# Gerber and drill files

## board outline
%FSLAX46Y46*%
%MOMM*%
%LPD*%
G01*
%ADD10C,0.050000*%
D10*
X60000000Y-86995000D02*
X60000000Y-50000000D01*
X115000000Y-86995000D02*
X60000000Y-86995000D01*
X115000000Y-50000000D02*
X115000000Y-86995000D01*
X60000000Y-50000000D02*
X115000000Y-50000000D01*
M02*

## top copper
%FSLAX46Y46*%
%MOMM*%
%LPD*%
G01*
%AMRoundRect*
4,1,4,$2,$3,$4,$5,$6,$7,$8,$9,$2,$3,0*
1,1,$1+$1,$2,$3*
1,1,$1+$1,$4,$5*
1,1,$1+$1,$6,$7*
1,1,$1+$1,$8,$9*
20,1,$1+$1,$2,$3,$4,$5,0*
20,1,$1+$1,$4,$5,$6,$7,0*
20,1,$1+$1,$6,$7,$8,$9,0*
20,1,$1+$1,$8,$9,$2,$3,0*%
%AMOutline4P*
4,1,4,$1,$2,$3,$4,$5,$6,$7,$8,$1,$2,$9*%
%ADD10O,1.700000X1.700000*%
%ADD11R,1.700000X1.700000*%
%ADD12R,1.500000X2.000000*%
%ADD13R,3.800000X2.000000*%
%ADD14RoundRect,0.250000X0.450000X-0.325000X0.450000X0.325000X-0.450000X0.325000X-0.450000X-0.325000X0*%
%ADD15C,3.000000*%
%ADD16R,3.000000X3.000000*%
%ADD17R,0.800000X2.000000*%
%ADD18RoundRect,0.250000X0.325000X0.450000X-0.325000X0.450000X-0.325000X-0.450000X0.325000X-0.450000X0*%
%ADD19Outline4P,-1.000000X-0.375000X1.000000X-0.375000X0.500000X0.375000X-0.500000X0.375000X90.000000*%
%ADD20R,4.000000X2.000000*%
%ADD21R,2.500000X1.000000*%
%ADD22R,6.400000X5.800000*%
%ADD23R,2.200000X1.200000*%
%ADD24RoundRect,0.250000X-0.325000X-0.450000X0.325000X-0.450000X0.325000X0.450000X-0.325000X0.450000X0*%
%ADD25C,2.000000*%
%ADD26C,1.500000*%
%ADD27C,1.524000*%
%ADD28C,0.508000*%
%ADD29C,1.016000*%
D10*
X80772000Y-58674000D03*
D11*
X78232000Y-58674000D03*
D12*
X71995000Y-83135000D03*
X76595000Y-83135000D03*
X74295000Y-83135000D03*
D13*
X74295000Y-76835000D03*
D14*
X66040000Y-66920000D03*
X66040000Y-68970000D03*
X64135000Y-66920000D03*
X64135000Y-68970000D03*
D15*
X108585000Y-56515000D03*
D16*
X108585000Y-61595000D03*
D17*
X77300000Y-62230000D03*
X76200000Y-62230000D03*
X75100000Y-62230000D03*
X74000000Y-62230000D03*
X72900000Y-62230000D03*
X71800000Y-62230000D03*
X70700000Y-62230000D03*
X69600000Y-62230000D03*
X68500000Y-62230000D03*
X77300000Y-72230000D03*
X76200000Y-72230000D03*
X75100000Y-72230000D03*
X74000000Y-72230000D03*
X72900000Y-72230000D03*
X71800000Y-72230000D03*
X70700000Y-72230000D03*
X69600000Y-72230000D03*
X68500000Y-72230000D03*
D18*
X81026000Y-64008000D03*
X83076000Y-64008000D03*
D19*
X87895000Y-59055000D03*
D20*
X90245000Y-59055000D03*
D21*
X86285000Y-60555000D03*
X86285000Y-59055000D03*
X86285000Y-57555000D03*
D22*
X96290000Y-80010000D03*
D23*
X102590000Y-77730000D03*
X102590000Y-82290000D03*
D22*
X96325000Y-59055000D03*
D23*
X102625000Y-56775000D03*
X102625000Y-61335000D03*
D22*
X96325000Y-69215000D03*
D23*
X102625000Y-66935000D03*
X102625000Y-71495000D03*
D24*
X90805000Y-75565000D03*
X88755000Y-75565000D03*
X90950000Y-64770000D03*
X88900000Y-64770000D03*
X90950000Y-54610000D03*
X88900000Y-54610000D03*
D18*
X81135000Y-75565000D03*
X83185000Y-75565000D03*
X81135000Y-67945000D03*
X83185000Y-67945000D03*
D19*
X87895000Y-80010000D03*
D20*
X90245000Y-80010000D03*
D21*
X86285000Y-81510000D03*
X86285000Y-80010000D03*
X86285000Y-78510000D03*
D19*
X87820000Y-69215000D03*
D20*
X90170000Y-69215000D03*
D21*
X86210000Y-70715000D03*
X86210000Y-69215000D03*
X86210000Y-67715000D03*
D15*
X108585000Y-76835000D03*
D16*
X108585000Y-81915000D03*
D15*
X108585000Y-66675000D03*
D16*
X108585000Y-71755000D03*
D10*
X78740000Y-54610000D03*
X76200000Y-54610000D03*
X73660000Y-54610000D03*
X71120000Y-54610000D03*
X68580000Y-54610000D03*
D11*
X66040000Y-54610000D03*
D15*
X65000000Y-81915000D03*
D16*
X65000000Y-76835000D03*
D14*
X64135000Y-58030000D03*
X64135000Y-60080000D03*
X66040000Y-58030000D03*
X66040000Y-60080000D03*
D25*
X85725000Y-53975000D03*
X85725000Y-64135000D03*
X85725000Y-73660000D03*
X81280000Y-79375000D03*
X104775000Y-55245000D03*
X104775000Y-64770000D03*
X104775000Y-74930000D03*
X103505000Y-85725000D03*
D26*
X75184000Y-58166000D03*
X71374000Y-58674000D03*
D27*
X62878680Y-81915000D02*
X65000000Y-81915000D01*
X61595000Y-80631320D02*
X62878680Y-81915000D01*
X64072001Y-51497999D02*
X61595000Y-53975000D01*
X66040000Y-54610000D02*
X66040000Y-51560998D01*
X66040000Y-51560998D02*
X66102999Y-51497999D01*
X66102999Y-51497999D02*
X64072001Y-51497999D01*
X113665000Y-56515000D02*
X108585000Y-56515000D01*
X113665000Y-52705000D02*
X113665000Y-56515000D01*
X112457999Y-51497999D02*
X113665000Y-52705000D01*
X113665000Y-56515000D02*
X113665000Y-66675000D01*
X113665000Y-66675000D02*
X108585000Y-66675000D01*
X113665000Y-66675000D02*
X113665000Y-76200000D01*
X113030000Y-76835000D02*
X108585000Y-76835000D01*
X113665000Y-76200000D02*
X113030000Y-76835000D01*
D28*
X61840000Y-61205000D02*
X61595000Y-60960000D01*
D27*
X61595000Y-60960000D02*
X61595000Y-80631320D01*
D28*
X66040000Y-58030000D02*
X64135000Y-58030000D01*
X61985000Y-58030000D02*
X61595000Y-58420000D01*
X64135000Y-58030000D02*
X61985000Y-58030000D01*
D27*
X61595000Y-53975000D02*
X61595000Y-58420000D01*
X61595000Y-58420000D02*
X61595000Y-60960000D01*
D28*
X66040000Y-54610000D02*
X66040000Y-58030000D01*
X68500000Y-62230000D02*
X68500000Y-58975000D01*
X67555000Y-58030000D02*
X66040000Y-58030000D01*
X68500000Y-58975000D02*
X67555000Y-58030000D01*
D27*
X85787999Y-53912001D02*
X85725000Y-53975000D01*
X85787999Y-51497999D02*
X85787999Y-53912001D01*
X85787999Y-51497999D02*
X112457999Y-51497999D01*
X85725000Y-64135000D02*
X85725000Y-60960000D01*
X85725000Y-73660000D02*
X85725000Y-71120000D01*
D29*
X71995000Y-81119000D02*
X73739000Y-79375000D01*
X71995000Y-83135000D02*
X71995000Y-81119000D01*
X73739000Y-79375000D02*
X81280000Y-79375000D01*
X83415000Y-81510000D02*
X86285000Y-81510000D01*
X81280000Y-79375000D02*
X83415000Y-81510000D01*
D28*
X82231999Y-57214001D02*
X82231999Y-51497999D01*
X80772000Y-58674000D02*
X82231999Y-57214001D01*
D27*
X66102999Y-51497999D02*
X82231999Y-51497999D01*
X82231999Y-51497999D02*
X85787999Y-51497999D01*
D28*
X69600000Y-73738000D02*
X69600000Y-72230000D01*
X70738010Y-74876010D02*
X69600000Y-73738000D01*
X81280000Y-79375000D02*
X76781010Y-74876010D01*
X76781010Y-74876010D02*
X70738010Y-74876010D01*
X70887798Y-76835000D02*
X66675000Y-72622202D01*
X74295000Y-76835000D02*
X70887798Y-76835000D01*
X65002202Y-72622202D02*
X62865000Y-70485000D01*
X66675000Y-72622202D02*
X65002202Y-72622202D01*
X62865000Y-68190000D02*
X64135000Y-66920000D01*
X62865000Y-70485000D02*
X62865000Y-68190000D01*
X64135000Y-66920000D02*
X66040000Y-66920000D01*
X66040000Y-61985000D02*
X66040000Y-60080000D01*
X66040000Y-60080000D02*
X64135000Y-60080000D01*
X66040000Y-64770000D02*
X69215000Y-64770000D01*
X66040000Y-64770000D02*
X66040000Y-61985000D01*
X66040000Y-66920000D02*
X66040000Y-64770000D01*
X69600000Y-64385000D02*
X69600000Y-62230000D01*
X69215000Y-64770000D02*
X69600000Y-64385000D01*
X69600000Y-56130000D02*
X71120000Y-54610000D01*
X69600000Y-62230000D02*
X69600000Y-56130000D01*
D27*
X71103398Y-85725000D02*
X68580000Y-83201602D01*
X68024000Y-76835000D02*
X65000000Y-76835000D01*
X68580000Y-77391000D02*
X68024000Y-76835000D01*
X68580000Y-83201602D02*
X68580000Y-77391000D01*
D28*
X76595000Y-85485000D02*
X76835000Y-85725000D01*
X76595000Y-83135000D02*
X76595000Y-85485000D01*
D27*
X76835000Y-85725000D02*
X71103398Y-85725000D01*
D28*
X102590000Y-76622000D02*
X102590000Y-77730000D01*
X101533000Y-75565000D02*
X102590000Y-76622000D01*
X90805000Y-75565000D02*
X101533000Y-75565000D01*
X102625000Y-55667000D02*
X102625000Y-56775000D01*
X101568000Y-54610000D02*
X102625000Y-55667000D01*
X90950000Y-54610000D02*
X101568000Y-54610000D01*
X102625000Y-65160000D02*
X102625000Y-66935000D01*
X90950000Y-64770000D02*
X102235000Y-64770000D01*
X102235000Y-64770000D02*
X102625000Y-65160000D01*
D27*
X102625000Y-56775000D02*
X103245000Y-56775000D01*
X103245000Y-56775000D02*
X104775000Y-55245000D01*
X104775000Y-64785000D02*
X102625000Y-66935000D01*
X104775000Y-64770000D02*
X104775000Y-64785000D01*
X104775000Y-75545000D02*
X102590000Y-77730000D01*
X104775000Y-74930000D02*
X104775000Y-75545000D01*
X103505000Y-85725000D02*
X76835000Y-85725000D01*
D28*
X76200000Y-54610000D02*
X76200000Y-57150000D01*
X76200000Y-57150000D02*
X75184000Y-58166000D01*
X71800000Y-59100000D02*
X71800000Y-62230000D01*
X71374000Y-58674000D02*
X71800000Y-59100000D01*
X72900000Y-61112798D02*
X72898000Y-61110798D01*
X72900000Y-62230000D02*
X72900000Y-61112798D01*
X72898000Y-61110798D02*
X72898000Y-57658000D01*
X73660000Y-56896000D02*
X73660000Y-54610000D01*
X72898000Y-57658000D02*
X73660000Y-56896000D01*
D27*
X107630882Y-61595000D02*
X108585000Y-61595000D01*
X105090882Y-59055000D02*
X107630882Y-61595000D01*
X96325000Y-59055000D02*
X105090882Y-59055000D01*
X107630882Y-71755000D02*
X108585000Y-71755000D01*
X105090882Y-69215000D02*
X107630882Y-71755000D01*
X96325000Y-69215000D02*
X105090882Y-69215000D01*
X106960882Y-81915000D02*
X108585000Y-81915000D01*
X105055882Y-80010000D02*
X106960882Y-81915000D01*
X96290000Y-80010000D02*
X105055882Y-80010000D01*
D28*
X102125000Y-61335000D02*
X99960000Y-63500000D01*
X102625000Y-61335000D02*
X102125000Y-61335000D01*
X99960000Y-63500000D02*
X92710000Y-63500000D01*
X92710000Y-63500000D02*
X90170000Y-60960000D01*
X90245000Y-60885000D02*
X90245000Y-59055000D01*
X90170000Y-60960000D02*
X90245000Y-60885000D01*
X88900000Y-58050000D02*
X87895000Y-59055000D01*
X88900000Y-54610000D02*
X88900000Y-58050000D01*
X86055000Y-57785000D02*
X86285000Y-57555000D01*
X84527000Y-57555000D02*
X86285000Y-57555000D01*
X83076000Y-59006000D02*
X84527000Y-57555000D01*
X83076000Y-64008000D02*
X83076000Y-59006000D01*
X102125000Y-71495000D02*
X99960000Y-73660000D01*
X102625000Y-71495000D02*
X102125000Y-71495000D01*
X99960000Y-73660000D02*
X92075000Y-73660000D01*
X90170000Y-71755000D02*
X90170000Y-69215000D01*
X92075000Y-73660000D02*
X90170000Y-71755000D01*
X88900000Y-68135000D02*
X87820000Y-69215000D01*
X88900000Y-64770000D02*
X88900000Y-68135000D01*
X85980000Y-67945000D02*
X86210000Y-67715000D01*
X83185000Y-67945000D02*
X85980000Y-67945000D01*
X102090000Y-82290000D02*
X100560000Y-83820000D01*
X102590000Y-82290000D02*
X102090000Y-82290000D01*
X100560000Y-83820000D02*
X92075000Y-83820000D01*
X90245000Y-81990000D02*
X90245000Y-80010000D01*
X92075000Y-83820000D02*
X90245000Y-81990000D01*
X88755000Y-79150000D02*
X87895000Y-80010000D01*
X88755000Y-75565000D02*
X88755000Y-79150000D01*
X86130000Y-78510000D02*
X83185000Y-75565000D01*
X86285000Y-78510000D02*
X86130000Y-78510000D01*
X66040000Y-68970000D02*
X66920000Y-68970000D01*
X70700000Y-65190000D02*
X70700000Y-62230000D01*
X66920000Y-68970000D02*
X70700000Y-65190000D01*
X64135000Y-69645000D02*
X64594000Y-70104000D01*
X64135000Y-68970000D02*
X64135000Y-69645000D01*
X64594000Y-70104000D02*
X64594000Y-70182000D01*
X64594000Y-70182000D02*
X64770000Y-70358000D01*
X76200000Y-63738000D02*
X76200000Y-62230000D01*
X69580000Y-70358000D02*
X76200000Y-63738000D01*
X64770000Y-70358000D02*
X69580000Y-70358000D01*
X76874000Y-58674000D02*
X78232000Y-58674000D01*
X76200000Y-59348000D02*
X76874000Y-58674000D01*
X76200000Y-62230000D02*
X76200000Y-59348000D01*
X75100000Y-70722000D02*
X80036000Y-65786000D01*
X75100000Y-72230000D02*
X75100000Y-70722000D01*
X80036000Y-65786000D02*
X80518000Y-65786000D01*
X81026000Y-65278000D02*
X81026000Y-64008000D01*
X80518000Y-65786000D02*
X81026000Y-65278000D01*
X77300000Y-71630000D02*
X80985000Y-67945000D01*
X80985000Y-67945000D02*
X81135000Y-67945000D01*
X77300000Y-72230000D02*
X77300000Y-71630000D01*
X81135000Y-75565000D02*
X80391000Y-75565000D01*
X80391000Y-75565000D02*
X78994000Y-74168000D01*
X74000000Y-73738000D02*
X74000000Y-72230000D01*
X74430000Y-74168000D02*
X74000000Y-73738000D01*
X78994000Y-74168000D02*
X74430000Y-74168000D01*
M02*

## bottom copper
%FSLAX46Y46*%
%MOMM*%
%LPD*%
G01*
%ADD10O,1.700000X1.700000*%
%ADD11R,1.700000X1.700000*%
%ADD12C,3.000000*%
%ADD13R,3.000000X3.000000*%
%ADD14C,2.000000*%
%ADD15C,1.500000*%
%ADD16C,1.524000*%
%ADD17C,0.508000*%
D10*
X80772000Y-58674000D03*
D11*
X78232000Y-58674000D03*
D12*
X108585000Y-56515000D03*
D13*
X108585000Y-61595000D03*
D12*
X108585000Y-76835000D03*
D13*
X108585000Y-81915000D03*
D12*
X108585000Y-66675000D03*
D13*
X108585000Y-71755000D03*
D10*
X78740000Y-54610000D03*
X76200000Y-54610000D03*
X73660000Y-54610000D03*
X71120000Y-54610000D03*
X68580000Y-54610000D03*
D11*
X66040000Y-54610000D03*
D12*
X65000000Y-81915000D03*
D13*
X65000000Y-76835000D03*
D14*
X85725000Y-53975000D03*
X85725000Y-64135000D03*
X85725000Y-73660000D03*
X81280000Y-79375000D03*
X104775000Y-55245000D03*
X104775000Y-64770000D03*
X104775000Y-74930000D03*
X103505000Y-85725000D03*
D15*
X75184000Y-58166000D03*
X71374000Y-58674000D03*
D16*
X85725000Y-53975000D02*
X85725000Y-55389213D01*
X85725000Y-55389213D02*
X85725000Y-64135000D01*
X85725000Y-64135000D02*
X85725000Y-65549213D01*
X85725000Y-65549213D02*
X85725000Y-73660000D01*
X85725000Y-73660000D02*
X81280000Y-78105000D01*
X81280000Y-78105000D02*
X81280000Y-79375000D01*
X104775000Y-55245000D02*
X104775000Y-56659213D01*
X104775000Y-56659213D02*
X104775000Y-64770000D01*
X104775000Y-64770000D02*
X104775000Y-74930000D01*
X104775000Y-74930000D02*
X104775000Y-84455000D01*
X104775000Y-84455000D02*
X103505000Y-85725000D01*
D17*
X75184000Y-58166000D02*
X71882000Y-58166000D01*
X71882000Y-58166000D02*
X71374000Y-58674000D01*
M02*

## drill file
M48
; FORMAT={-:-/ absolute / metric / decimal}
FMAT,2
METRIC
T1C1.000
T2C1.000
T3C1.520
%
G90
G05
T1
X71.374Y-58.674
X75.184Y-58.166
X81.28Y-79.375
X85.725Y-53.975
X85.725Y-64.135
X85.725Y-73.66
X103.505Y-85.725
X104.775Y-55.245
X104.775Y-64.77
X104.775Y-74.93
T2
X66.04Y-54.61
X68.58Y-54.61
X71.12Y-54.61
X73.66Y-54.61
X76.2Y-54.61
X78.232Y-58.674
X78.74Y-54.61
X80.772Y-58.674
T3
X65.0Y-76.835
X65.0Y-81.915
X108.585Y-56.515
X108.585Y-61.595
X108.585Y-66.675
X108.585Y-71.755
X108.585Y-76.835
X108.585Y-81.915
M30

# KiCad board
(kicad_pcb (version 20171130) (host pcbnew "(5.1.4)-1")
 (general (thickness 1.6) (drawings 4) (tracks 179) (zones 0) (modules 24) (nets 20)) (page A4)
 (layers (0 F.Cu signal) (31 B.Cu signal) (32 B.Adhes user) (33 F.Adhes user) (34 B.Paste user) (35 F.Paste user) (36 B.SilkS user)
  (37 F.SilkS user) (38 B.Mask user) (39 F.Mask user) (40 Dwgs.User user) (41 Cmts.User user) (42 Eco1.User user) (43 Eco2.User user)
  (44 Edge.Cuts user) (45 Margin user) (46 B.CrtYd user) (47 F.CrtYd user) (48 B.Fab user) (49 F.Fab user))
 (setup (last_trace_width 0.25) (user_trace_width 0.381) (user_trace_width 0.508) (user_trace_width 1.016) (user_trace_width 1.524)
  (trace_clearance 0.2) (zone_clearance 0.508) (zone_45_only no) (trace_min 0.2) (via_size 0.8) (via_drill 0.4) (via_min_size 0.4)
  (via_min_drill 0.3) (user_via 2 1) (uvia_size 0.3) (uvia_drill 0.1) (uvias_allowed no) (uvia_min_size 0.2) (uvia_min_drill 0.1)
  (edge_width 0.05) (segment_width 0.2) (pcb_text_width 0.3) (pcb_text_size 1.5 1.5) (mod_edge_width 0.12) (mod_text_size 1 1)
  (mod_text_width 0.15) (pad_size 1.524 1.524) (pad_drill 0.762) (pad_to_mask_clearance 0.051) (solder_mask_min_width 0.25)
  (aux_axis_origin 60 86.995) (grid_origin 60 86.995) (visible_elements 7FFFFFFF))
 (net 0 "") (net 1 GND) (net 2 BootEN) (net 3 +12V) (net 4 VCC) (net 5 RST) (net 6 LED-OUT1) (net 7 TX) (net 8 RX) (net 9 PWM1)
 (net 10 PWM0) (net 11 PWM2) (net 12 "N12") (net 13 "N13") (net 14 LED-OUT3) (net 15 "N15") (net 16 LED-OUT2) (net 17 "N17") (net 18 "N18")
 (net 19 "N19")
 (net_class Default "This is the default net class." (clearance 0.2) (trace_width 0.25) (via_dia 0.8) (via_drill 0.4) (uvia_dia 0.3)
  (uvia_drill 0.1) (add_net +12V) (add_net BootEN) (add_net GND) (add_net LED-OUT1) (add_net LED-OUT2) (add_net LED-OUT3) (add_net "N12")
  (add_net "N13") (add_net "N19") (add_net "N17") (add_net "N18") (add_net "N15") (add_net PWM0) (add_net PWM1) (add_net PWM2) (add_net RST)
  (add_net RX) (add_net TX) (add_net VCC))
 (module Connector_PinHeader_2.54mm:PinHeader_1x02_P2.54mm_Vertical (layer F.Cu) (at 78.232 58.674 90)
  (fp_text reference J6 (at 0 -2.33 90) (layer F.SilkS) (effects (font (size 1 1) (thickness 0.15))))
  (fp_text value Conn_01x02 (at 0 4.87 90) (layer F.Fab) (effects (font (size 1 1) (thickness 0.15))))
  (pad 2 thru_hole oval (at 0 2.54 90) (size 1.7 1.7) (drill 1) (layers *.Cu *.Mask) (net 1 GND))
  (pad 1 thru_hole rect (at 0 0 90) (size 1.7 1.7) (drill 1) (layers *.Cu *.Mask) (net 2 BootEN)))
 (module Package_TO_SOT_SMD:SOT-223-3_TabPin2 (layer F.Cu) (at 74.295 79.985 90)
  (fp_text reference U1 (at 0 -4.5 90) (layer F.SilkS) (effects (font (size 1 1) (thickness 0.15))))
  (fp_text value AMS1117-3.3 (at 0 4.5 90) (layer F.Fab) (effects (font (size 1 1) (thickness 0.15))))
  (pad 1 smd rect (at -3.15 -2.3 90) (size 2 1.5) (layers F.Cu F.Paste F.Mask) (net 1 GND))
  (pad 3 smd rect (at -3.15 2.3 90) (size 2 1.5) (layers F.Cu F.Paste F.Mask) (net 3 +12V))
  (pad 2 smd rect (at -3.15 0 90) (size 2 1.5) (layers F.Cu F.Paste F.Mask) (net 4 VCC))
  (pad 2 smd rect (at 3.15 0 90) (size 2 3.8) (layers F.Cu F.Paste F.Mask) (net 4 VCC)))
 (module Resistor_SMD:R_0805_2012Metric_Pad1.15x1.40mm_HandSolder (layer F.Cu) (at 66.04 67.945 90)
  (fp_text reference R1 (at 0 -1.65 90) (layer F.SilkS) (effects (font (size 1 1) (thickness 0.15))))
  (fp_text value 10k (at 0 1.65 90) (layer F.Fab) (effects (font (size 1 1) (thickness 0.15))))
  (pad 2 smd roundrect (at 1.025 0 90) (size 1.15 1.4) (layers F.Cu F.Paste F.Mask) (roundrect_rratio 0.217391) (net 4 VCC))
  (pad 1 smd roundrect (at -1.025 0 90) (size 1.15 1.4) (layers F.Cu F.Paste F.Mask) (roundrect_rratio 0.217391) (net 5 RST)))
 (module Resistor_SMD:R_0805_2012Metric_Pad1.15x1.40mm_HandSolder (layer F.Cu) (at 64.135 67.945 90)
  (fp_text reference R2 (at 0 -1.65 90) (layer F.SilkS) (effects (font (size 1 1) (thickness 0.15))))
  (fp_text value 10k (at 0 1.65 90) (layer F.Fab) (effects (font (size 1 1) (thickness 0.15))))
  (pad 2 smd roundrect (at 1.025 0 90) (size 1.15 1.4) (layers F.Cu F.Paste F.Mask) (roundrect_rratio 0.217391) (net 4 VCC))
  (pad 1 smd roundrect (at -1.025 0 90) (size 1.15 1.4) (layers F.Cu F.Paste F.Mask) (roundrect_rratio 0.217391) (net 2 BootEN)))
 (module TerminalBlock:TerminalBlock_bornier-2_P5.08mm (layer F.Cu) (at 108.585 61.595 90)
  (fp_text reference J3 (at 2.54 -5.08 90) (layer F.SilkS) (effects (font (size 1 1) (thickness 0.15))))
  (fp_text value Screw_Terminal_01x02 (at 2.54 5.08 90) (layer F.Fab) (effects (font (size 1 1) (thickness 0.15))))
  (pad 2 thru_hole circle (at 5.08 0 90) (size 3 3) (drill 1.52) (layers *.Cu *.Mask) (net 1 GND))
  (pad 1 thru_hole rect (at 0 0 90) (size 3 3) (drill 1.52) (layers *.Cu *.Mask) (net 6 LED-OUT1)))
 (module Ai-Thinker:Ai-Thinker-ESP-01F (layer F.Cu) (at 72.4 67.23 90)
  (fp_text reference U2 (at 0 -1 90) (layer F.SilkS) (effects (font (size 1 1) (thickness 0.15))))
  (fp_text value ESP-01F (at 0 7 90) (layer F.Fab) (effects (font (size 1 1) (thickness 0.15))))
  (pad 18 smd rect (at 5 4.9 90) (size 2 0.8) (layers F.Cu F.Paste F.Mask))
  (pad 17 smd rect (at 5 3.8 90) (size 2 0.8) (layers F.Cu F.Paste F.Mask) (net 2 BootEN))
  (pad 16 smd rect (at 5 2.7 90) (size 2 0.8) (layers F.Cu F.Paste F.Mask))
  (pad 15 smd rect (at 5 1.6 90) (size 2 0.8) (layers F.Cu F.Paste F.Mask))
  (pad 14 smd rect (at 5 0.5 90) (size 2 0.8) (layers F.Cu F.Paste F.Mask) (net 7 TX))
  (pad 13 smd rect (at 5 -0.6 90) (size 2 0.8) (layers F.Cu F.Paste F.Mask) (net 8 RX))
  (pad 12 smd rect (at 5 -1.7 90) (size 2 0.8) (layers F.Cu F.Paste F.Mask) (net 5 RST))
  (pad 11 smd rect (at 5 -2.8 90) (size 2 0.8) (layers F.Cu F.Paste F.Mask) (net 4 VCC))
  (pad 10 smd rect (at 5 -3.9 90) (size 2 0.8) (layers F.Cu F.Paste F.Mask) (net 1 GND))
  (pad 9 smd rect (at -5 4.9 90) (size 2 0.8) (layers F.Cu F.Paste F.Mask) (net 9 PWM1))
  (pad 8 smd rect (at -5 3.8 90) (size 2 0.8) (layers F.Cu F.Paste F.Mask))
  (pad 7 smd rect (at -5 2.7 90) (size 2 0.8) (layers F.Cu F.Paste F.Mask) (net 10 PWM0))
  (pad 6 smd rect (at -5 1.6 90) (size 2 0.8) (layers F.Cu F.Paste F.Mask) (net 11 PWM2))
  (pad 5 smd rect (at -5 0.5 90) (size 2 0.8) (layers F.Cu F.Paste F.Mask))
  (pad 4 smd rect (at -5 -0.6 90) (size 2 0.8) (layers F.Cu F.Paste F.Mask))
  (pad 3 smd rect (at -5 -1.7 90) (size 2 0.8) (layers F.Cu F.Paste F.Mask))
  (pad 2 smd rect (at -5 -2.8 90) (size 2 0.8) (layers F.Cu F.Paste F.Mask) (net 1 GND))
  (pad 1 smd rect (at -5 -3.9 90) (size 2 0.8) (layers F.Cu F.Paste F.Mask)))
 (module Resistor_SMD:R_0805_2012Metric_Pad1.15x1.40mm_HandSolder (layer F.Cu) (at 82.051 64.008 180)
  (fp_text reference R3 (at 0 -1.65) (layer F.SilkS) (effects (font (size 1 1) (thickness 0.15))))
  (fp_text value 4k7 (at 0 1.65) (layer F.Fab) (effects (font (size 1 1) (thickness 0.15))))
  (pad 2 smd roundrect (at 1.025 0 180) (size 1.15 1.4) (layers F.Cu F.Paste F.Mask) (roundrect_rratio 0.217391) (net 10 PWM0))
  (pad 1 smd roundrect (at -1.025 0 180) (size 1.15 1.4) (layers F.Cu F.Paste F.Mask) (roundrect_rratio 0.217391) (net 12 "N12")))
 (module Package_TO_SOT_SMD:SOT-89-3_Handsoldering (layer F.Cu) (at 88.265 59.055)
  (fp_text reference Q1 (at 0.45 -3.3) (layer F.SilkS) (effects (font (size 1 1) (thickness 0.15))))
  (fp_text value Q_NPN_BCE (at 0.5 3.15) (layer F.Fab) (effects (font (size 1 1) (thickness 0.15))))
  (pad 2 smd trapezoid (at -0.37 0 90) (size 1.5 0.75) (rect_delta 0 0.5) (layers F.Cu F.Paste F.Mask) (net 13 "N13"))
  (pad 2 smd rect (at 1.98 0 270) (size 2 4) (layers F.Cu F.Paste F.Mask) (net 13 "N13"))
  (pad 3 smd rect (at -1.98 1.5 270) (size 1 2.5) (layers F.Cu F.Paste F.Mask) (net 1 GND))
  (pad 2 smd rect (at -1.98 0 270) (size 1 2.5) (layers F.Cu F.Paste F.Mask) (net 13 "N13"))
  (pad 1 smd rect (at -1.98 -1.5 270) (size 1 2.5) (layers F.Cu F.Paste F.Mask) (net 12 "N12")))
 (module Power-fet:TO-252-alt (layer F.Cu) (at 98.39 80.01 180)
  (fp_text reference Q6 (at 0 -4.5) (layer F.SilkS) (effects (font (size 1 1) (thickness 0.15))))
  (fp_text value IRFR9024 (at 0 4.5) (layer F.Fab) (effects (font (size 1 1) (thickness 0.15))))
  (pad "" smd rect (at 0.425 1.525 180) (size 3.05 2.75) (layers F.Paste))
  (pad "" smd rect (at 3.775 -1.525 180) (size 3.05 2.75) (layers F.Paste))
  (pad "" smd rect (at 0.425 -1.525 180) (size 3.05 2.75) (layers F.Paste))
  (pad "" smd rect (at 3.775 1.525 180) (size 3.05 2.75) (layers F.Paste))
  (pad 3 smd rect (at 2.1 0 180) (size 6.4 5.8) (layers F.Cu F.Mask) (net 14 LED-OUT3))
  (pad 1 smd rect (at -4.2 2.28 180) (size 2.2 1.2) (layers F.Cu F.Paste F.Mask) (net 3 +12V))
  (pad 2 smd rect (at -4.2 -2.28 180) (size 2.2 1.2) (layers F.Cu F.Paste F.Mask) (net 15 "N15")))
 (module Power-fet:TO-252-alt (layer F.Cu) (at 98.425 59.055 180)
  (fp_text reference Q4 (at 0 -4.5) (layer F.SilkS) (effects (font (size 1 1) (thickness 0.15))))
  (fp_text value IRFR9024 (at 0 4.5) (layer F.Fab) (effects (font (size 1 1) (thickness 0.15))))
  (pad "" smd rect (at 0.425 1.525 180) (size 3.05 2.75) (layers F.Paste))
  (pad "" smd rect (at 3.775 -1.525 180) (size 3.05 2.75) (layers F.Paste))
  (pad "" smd rect (at 0.425 -1.525 180) (size 3.05 2.75) (layers F.Paste))
  (pad "" smd rect (at 3.775 1.525 180) (size 3.05 2.75) (layers F.Paste))
  (pad 3 smd rect (at 2.1 0 180) (size 6.4 5.8) (layers F.Cu F.Mask) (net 6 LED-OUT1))
  (pad 1 smd rect (at -4.2 2.28 180) (size 2.2 1.2) (layers F.Cu F.Paste F.Mask) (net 3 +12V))
  (pad 2 smd rect (at -4.2 -2.28 180) (size 2.2 1.2) (layers F.Cu F.Paste F.Mask) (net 13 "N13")))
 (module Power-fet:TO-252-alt (layer F.Cu) (at 98.425 69.215 180)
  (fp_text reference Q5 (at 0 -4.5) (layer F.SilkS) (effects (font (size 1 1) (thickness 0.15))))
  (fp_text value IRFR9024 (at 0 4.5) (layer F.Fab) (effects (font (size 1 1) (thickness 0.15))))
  (pad "" smd rect (at 0.425 1.525 180) (size 3.05 2.75) (layers F.Paste))
  (pad "" smd rect (at 3.775 -1.525 180) (size 3.05 2.75) (layers F.Paste))
  (pad "" smd rect (at 0.425 -1.525 180) (size 3.05 2.75) (layers F.Paste))
  (pad "" smd rect (at 3.775 1.525 180) (size 3.05 2.75) (layers F.Paste))
  (pad 3 smd rect (at 2.1 0 180) (size 6.4 5.8) (layers F.Cu F.Mask) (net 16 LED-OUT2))
  (pad 1 smd rect (at -4.2 2.28 180) (size 2.2 1.2) (layers F.Cu F.Paste F.Mask) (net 3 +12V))
  (pad 2 smd rect (at -4.2 -2.28 180) (size 2.2 1.2) (layers F.Cu F.Paste F.Mask) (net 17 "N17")))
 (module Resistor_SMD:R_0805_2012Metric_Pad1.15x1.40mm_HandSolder (layer F.Cu) (at 89.78 75.565)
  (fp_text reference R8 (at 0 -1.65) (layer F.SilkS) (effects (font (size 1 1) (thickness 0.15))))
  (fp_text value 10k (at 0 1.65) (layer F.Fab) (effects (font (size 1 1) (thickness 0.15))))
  (pad 2 smd roundrect (at 1.025 0) (size 1.15 1.4) (layers F.Cu F.Paste F.Mask) (roundrect_rratio 0.217391) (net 3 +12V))
  (pad 1 smd roundrect (at -1.025 0) (size 1.15 1.4) (layers F.Cu F.Paste F.Mask) (roundrect_rratio 0.217391) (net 15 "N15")))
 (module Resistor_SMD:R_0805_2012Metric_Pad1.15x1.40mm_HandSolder (layer F.Cu) (at 89.925 64.77)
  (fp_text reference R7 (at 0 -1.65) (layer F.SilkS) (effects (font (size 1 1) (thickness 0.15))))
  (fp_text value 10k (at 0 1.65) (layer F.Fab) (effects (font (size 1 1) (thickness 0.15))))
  (pad 2 smd roundrect (at 1.025 0) (size 1.15 1.4) (layers F.Cu F.Paste F.Mask) (roundrect_rratio 0.217391) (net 3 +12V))
  (pad 1 smd roundrect (at -1.025 0) (size 1.15 1.4) (layers F.Cu F.Paste F.Mask) (roundrect_rratio 0.217391) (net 17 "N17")))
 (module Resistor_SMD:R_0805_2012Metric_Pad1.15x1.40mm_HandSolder (layer F.Cu) (at 89.925 54.61)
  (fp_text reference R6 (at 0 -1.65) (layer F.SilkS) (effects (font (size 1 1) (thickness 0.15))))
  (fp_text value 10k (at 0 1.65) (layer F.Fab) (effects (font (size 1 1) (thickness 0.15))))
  (pad 2 smd roundrect (at 1.025 0) (size 1.15 1.4) (layers F.Cu F.Paste F.Mask) (roundrect_rratio 0.217391) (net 3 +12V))
  (pad 1 smd roundrect (at -1.025 0) (size 1.15 1.4) (layers F.Cu F.Paste F.Mask) (roundrect_rratio 0.217391) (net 13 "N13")))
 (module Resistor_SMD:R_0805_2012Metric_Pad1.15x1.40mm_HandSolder (layer F.Cu) (at 82.16 75.565 180)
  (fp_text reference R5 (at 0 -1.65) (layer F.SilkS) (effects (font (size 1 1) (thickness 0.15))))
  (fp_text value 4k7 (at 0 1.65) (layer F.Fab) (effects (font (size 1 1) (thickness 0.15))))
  (pad 2 smd roundrect (at 1.025 0 180) (size 1.15 1.4) (layers F.Cu F.Paste F.Mask) (roundrect_rratio 0.217391) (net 11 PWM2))
  (pad 1 smd roundrect (at -1.025 0 180) (size 1.15 1.4) (layers F.Cu F.Paste F.Mask) (roundrect_rratio 0.217391) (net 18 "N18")))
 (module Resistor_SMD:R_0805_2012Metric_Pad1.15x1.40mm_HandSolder (layer F.Cu) (at 82.16 67.945 180)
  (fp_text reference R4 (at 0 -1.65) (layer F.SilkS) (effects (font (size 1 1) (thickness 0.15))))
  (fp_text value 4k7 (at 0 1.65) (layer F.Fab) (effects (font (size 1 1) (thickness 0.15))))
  (pad 2 smd roundrect (at 1.025 0 180) (size 1.15 1.4) (layers F.Cu F.Paste F.Mask) (roundrect_rratio 0.217391) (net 9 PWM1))
  (pad 1 smd roundrect (at -1.025 0 180) (size 1.15 1.4) (layers F.Cu F.Paste F.Mask) (roundrect_rratio 0.217391) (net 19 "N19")))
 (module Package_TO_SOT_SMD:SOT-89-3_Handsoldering (layer F.Cu) (at 88.265 80.01)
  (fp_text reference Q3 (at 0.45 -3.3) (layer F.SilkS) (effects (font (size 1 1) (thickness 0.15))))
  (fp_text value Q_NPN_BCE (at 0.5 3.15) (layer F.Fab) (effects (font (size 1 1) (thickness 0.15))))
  (pad 2 smd trapezoid (at -0.37 0 90) (size 1.5 0.75) (rect_delta 0 0.5) (layers F.Cu F.Paste F.Mask) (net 15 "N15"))
  (pad 2 smd rect (at 1.98 0 270) (size 2 4) (layers F.Cu F.Paste F.Mask) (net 15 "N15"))
  (pad 3 smd rect (at -1.98 1.5 270) (size 1 2.5) (layers F.Cu F.Paste F.Mask) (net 1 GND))
  (pad 2 smd rect (at -1.98 0 270) (size 1 2.5) (layers F.Cu F.Paste F.Mask) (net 15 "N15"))
  (pad 1 smd rect (at -1.98 -1.5 270) (size 1 2.5) (layers F.Cu F.Paste F.Mask) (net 18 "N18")))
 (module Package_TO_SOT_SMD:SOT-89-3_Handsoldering (layer F.Cu) (at 88.19 69.215)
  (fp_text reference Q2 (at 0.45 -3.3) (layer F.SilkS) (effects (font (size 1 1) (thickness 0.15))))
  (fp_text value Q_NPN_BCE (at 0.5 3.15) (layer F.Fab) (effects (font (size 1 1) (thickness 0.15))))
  (pad 2 smd trapezoid (at -0.37 0 90) (size 1.5 0.75) (rect_delta 0 0.5) (layers F.Cu F.Paste F.Mask) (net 17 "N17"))
  (pad 2 smd rect (at 1.98 0 270) (size 2 4) (layers F.Cu F.Paste F.Mask) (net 17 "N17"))
  (pad 3 smd rect (at -1.98 1.5 270) (size 1 2.5) (layers F.Cu F.Paste F.Mask) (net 1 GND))
  (pad 2 smd rect (at -1.98 0 270) (size 1 2.5) (layers F.Cu F.Paste F.Mask) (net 17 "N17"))
  (pad 1 smd rect (at -1.98 -1.5 270) (size 1 2.5) (layers F.Cu F.Paste F.Mask) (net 19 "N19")))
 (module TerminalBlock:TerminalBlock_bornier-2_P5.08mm (layer F.Cu) (at 108.585 81.915 90)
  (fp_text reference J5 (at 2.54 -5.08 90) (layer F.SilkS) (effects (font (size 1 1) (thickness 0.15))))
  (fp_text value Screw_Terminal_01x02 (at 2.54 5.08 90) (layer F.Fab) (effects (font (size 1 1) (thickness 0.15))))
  (pad 2 thru_hole circle (at 5.08 0 90) (size 3 3) (drill 1.52) (layers *.Cu *.Mask) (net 1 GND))
  (pad 1 thru_hole rect (at 0 0 90) (size 3 3) (drill 1.52) (layers *.Cu *.Mask) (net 14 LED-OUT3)))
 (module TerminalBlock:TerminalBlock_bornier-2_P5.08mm (layer F.Cu) (at 108.585 71.755 90)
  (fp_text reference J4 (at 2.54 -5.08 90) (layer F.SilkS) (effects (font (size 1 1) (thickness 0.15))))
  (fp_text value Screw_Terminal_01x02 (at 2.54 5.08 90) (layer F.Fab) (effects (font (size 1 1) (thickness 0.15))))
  (pad 2 thru_hole circle (at 5.08 0 90) (size 3 3) (drill 1.52) (layers *.Cu *.Mask) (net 1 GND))
  (pad 1 thru_hole rect (at 0 0 90) (size 3 3) (drill 1.52) (layers *.Cu *.Mask) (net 16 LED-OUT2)))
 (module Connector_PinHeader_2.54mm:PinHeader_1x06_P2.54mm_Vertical (layer F.Cu) (at 66.04 54.61 90)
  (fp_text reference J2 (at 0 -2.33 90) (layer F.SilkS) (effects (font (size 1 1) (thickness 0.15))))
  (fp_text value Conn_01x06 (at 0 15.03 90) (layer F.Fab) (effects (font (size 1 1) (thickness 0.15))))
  (pad 6 thru_hole oval (at 0 12.7 90) (size 1.7 1.7) (drill 1) (layers *.Cu *.Mask))
  (pad 5 thru_hole oval (at 0 10.16 90) (size 1.7 1.7) (drill 1) (layers *.Cu *.Mask) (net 8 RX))
  (pad 4 thru_hole oval (at 0 7.62 90) (size 1.7 1.7) (drill 1) (layers *.Cu *.Mask) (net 7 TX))
  (pad 3 thru_hole oval (at 0 5.08 90) (size 1.7 1.7) (drill 1) (layers *.Cu *.Mask) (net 4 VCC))
  (pad 2 thru_hole oval (at 0 2.54 90) (size 1.7 1.7) (drill 1) (layers *.Cu *.Mask))
  (pad 1 thru_hole rect (at 0 0 90) (size 1.7 1.7) (drill 1) (layers *.Cu *.Mask) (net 1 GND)))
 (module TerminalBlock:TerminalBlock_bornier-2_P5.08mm (layer F.Cu) (at 65 76.835 270)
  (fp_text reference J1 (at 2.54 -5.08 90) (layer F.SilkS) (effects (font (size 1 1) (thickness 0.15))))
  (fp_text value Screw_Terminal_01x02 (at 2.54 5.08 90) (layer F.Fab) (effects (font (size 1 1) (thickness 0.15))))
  (pad 2 thru_hole circle (at 5.08 0 270) (size 3 3) (drill 1.52) (layers *.Cu *.Mask) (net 1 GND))
  (pad 1 thru_hole rect (at 0 0 270) (size 3 3) (drill 1.52) (layers *.Cu *.Mask) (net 3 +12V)))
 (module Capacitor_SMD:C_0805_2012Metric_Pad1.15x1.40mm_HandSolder (layer F.Cu) (at 64.135 59.055 90)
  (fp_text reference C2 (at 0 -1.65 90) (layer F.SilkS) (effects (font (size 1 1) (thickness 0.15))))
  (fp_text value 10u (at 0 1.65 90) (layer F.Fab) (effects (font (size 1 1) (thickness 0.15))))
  (pad 2 smd roundrect (at 1.025 0 90) (size 1.15 1.4) (layers F.Cu F.Paste F.Mask) (roundrect_rratio 0.217391) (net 1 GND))
  (pad 1 smd roundrect (at -1.025 0 90) (size 1.15 1.4) (layers F.Cu F.Paste F.Mask) (roundrect_rratio 0.217391) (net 4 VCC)))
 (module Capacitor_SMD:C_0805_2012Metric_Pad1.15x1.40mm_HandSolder (layer F.Cu) (at 66.04 59.055 90)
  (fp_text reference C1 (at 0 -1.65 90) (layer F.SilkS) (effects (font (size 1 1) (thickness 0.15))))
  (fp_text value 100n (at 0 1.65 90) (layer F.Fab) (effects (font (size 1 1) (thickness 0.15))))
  (pad 2 smd roundrect (at 1.025 0 90) (size 1.15 1.4) (layers F.Cu F.Paste F.Mask) (roundrect_rratio 0.217391) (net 1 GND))
  (pad 1 smd roundrect (at -1.025 0 90) (size 1.15 1.4) (layers F.Cu F.Paste F.Mask) (roundrect_rratio 0.217391) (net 4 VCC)))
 (gr_line (start 60 86.995) (end 60 50) (layer Edge.Cuts) (width 0.05))
 (gr_line (start 115 86.995) (end 60 86.995) (layer Edge.Cuts) (width 0.05))
 (gr_line (start 115 50) (end 115 86.995) (layer Edge.Cuts) (width 0.05))
 (gr_line (start 60 50) (end 115 50) (layer Edge.Cuts) (width 0.05))
 (segment (start 62.87868 81.915) (end 65 81.915) (width 1.524) (layer F.Cu) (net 1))
 (segment (start 61.595 80.63132) (end 62.87868 81.915) (width 1.524) (layer F.Cu) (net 1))
 (segment (start 64.072001 51.497999) (end 61.595 53.975) (width 1.524) (layer F.Cu) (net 1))
 (segment (start 66.04 54.61) (end 66.04 51.560998) (width 1.524) (layer F.Cu) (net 1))
 (segment (start 66.04 51.560998) (end 66.102999 51.497999) (width 1.524) (layer F.Cu) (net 1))
 (segment (start 66.102999 51.497999) (end 64.072001 51.497999) (width 1.524) (layer F.Cu) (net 1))
 (segment (start 113.665 56.515) (end 108.585 56.515) (width 1.524) (layer F.Cu) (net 1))
 (segment (start 113.665 52.705) (end 113.665 56.515) (width 1.524) (layer F.Cu) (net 1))
 (segment (start 112.457999 51.497999) (end 113.665 52.705) (width 1.524) (layer F.Cu) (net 1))
 (segment (start 113.665 56.515) (end 113.665 66.675) (width 1.524) (layer F.Cu) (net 1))
 (segment (start 113.665 66.675) (end 108.585 66.675) (width 1.524) (layer F.Cu) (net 1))
 (segment (start 113.665 66.675) (end 113.665 76.2) (width 1.524) (layer F.Cu) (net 1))
 (segment (start 113.03 76.835) (end 108.585 76.835) (width 1.524) (layer F.Cu) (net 1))
 (segment (start 113.665 76.2) (end 113.03 76.835) (width 1.524) (layer F.Cu) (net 1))
 (segment (start 61.84 61.205) (end 61.595 60.96) (width 0.508) (layer F.Cu) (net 1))
 (segment (start 61.595 60.96) (end 61.595 80.63132) (width 1.524) (layer F.Cu) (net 1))
 (segment (start 66.04 58.03) (end 64.135 58.03) (width 0.508) (layer F.Cu) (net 1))
 (segment (start 61.985 58.03) (end 61.595 58.42) (width 0.508) (layer F.Cu) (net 1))
 (segment (start 64.135 58.03) (end 61.985 58.03) (width 0.508) (layer F.Cu) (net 1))
 (segment (start 61.595 53.975) (end 61.595 58.42) (width 1.524) (layer F.Cu) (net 1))
 (segment (start 61.595 58.42) (end 61.595 60.96) (width 1.524) (layer F.Cu) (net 1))
 (segment (start 66.04 54.61) (end 66.04 58.03) (width 0.508) (layer F.Cu) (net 1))
 (segment (start 68.5 62.23) (end 68.5 58.975) (width 0.508) (layer F.Cu) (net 1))
 (segment (start 67.555 58.03) (end 66.04 58.03) (width 0.508) (layer F.Cu) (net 1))
 (segment (start 68.5 58.975) (end 67.555 58.03) (width 0.508) (layer F.Cu) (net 1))
 (via (at 85.725 53.975) (size 2) (drill 1) (layers F.Cu B.Cu) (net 1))
 (segment (start 85.787999 53.912001) (end 85.725 53.975) (width 1.524) (layer F.Cu) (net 1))
 (segment (start 85.787999 51.497999) (end 85.787999 53.912001) (width 1.524) (layer F.Cu) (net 1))
 (segment (start 85.787999 51.497999) (end 112.457999 51.497999) (width 1.524) (layer F.Cu) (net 1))
 (segment (start 85.725 53.975) (end 85.725 55.389213) (width 1.524) (layer B.Cu) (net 1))
 (via (at 85.725 64.135) (size 2) (drill 1) (layers F.Cu B.Cu) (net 1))
 (segment (start 85.725 55.389213) (end 85.725 64.135) (width 1.524) (layer B.Cu) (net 1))
 (segment (start 85.725 64.135) (end 85.725 60.96) (width 1.524) (layer F.Cu) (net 1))
 (segment (start 85.725 64.135) (end 85.725 65.549213) (width 1.524) (layer B.Cu) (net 1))
 (via (at 85.725 73.66) (size 2) (drill 1) (layers F.Cu B.Cu) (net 1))
 (segment (start 85.725 65.549213) (end 85.725 73.66) (width 1.524) (layer B.Cu) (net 1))
 (segment (start 85.725 73.66) (end 85.725 71.12) (width 1.524) (layer F.Cu) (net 1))
 (segment (start 85.725 73.66) (end 81.28 78.105) (width 1.524) (layer B.Cu) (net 1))
 (via (at 81.28 79.375) (size 2) (drill 1) (layers F.Cu B.Cu) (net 1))
 (segment (start 81.28 78.105) (end 81.28 79.375) (width 1.524) (layer B.Cu) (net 1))
 (segment (start 71.995 81.119) (end 73.739 79.375) (width 1.016) (layer F.Cu) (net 1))
 (segment (start 71.995 83.135) (end 71.995 81.119) (width 1.016) (layer F.Cu) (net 1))
 (segment (start 73.739 79.375) (end 81.28 79.375) (width 1.016) (layer F.Cu) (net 1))
 (segment (start 83.415 81.51) (end 86.285 81.51) (width 1.016) (layer F.Cu) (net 1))
 (segment (start 81.28 79.375) (end 83.415 81.51) (width 1.016) (layer F.Cu) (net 1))
 (segment (start 82.231999 57.214001) (end 82.231999 51.497999) (width 0.508) (layer F.Cu) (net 1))
 (segment (start 80.772 58.674) (end 82.231999 57.214001) (width 0.508) (layer F.Cu) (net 1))
 (segment (start 66.102999 51.497999) (end 82.231999 51.497999) (width 1.524) (layer F.Cu) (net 1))
 (segment (start 82.231999 51.497999) (end 85.787999 51.497999) (width 1.524) (layer F.Cu) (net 1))
 (segment (start 69.6 73.738) (end 69.6 72.23) (width 0.508) (layer F.Cu) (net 1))
 (segment (start 70.73801 74.87601) (end 69.6 73.738) (width 0.508) (layer F.Cu) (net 1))
 (segment (start 81.28 79.375) (end 76.78101 74.87601) (width 0.508) (layer F.Cu) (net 1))
 (segment (start 76.78101 74.87601) (end 70.73801 74.87601) (width 0.508) (layer F.Cu) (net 1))
 (segment (start 70.887798 76.835) (end 66.675 72.622202) (width 0.508) (layer F.Cu) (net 4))
 (segment (start 74.295 76.835) (end 70.887798 76.835) (width 0.508) (layer F.Cu) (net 4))
 (segment (start 65.002202 72.622202) (end 62.865 70.485) (width 0.508) (layer F.Cu) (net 4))
 (segment (start 66.675 72.622202) (end 65.002202 72.622202) (width 0.508) (layer F.Cu) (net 4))
 (segment (start 62.865 68.19) (end 64.135 66.92) (width 0.508) (layer F.Cu) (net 4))
 (segment (start 62.865 70.485) (end 62.865 68.19) (width 0.508) (layer F.Cu) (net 4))
 (segment (start 64.135 66.92) (end 66.04 66.92) (width 0.508) (layer F.Cu) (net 4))
 (segment (start 66.04 61.985) (end 66.04 60.08) (width 0.508) (layer F.Cu) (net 4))
 (segment (start 66.04 60.08) (end 64.135 60.08) (width 0.508) (layer F.Cu) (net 4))
 (segment (start 66.04 64.77) (end 69.215 64.77) (width 0.508) (layer F.Cu) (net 4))
 (segment (start 66.04 64.77) (end 66.04 61.985) (width 0.508) (layer F.Cu) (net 4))
 (segment (start 66.04 66.92) (end 66.04 64.77) (width 0.508) (layer F.Cu) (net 4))
 (segment (start 69.6 64.385) (end 69.6 62.23) (width 0.508) (layer F.Cu) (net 4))
 (segment (start 69.215 64.77) (end 69.6 64.385) (width 0.508) (layer F.Cu) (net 4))
 (segment (start 69.6 56.13) (end 71.12 54.61) (width 0.508) (layer F.Cu) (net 4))
 (segment (start 69.6 62.23) (end 69.6 56.13) (width 0.508) (layer F.Cu) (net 4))
 (segment (start 71.103398 85.725) (end 68.58 83.201602) (width 1.524) (layer F.Cu) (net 3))
 (segment (start 68.024 76.835) (end 65 76.835) (width 1.524) (layer F.Cu) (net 3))
 (segment (start 68.58 77.391) (end 68.024 76.835) (width 1.524) (layer F.Cu) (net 3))
 (segment (start 68.58 83.201602) (end 68.58 77.391) (width 1.524) (layer F.Cu) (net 3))
 (segment (start 76.595 85.485) (end 76.835 85.725) (width 0.508) (layer F.Cu) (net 3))
 (segment (start 76.595 83.135) (end 76.595 85.485) (width 0.508) (layer F.Cu) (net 3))
 (segment (start 76.835 85.725) (end 71.103398 85.725) (width 1.524) (layer F.Cu) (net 3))
 (segment (start 102.59 76.622) (end 102.59 77.73) (width 0.508) (layer F.Cu) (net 3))
 (segment (start 101.533 75.565) (end 102.59 76.622) (width 0.508) (layer F.Cu) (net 3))
 (segment (start 90.805 75.565) (end 101.533 75.565) (width 0.508) (layer F.Cu) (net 3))
 (segment (start 102.625 55.667) (end 102.625 56.775) (width 0.508) (layer F.Cu) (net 3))
 (segment (start 101.568 54.61) (end 102.625 55.667) (width 0.508) (layer F.Cu) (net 3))
 (segment (start 90.95 54.61) (end 101.568 54.61) (width 0.508) (layer F.Cu) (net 3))
 (segment (start 102.625 65.16) (end 102.625 66.935) (width 0.508) (layer F.Cu) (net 3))
 (segment (start 90.95 64.77) (end 102.235 64.77) (width 0.508) (layer F.Cu) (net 3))
 (segment (start 102.235 64.77) (end 102.625 65.16) (width 0.508) (layer F.Cu) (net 3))
 (segment (start 102.625 56.775) (end 103.245 56.775) (width 1.524) (layer F.Cu) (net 3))
 (segment (start 103.245 56.775) (end 104.775 55.245) (width 1.524) (layer F.Cu) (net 3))
 (via (at 104.775 55.245) (size 2) (drill 1) (layers F.Cu B.Cu) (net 3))
 (segment (start 104.775 55.245) (end 104.775 56.659213) (width 1.524) (layer B.Cu) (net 3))
 (via (at 104.775 64.77) (size 2) (drill 1) (layers F.Cu B.Cu) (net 3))
 (segment (start 104.775 56.659213) (end 104.775 64.77) (width 1.524) (layer B.Cu) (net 3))
 (segment (start 104.775 64.785) (end 102.625 66.935) (width 1.524) (layer F.Cu) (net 3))
 (segment (start 104.775 64.77) (end 104.775 64.785) (width 1.524) (layer F.Cu) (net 3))
 (via (at 104.775 74.93) (size 2) (drill 1) (layers F.Cu B.Cu) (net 3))
 (segment (start 104.775 64.77) (end 104.775 74.93) (width 1.524) (layer B.Cu) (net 3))
 (segment (start 104.775 75.545) (end 102.59 77.73) (width 1.524) (layer F.Cu) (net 3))
 (segment (start 104.775 74.93) (end 104.775 75.545) (width 1.524) (layer F.Cu) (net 3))
 (via (at 103.505 85.725) (size 2) (drill 1) (layers F.Cu B.Cu) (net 3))
 (segment (start 104.775 74.93) (end 104.775 84.455) (width 1.524) (layer B.Cu) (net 3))
 (segment (start 104.775 84.455) (end 103.505 85.725) (width 1.524) (layer B.Cu) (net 3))
 (segment (start 103.505 85.725) (end 76.835 85.725) (width 1.524) (layer F.Cu) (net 3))
 (via (at 75.184 58.166) (size 1.5) (drill 1) (layers F.Cu B.Cu) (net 8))
 (segment (start 76.2 54.61) (end 76.2 57.15) (width 0.508) (layer F.Cu) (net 8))
 (segment (start 76.2 57.15) (end 75.184 58.166) (width 0.508) (layer F.Cu) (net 8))
 (via (at 71.374 58.674) (size 1.5) (drill 1) (layers F.Cu B.Cu) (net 8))
 (segment (start 75.184 58.166) (end 71.882 58.166) (width 0.508) (layer B.Cu) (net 8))
 (segment (start 71.882 58.166) (end 71.374 58.674) (width 0.508) (layer B.Cu) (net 8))
 (segment (start 71.8 59.1) (end 71.8 62.23) (width 0.508) (layer F.Cu) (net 8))
 (segment (start 71.374 58.674) (end 71.8 59.1) (width 0.508) (layer F.Cu) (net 8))
 (segment (start 72.9 61.112798) (end 72.898 61.110798) (width 0.508) (layer F.Cu) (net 7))
 (segment (start 72.9 62.23) (end 72.9 61.112798) (width 0.508) (layer F.Cu) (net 7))
 (segment (start 72.898 61.110798) (end 72.898 57.658) (width 0.508) (layer F.Cu) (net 7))
 (segment (start 73.66 56.896) (end 73.66 54.61) (width 0.508) (layer F.Cu) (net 7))
 (segment (start 72.898 57.658) (end 73.66 56.896) (width 0.508) (layer F.Cu) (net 7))
 (segment (start 107.630882 61.595) (end 108.585 61.595) (width 1.524) (layer F.Cu) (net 6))
 (segment (start 105.090882 59.055) (end 107.630882 61.595) (width 1.524) (layer F.Cu) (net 6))
 (segment (start 96.325 59.055) (end 105.090882 59.055) (width 1.524) (layer F.Cu) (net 6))
 (segment (start 107.630882 71.755) (end 108.585 71.755) (width 1.524) (layer F.Cu) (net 16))
 (segment (start 105.090882 69.215) (end 107.630882 71.755) (width 1.524) (layer F.Cu) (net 16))
 (segment (start 96.325 69.215) (end 105.090882 69.215) (width 1.524) (layer F.Cu) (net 16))
 (segment (start 106.960882 81.915) (end 108.585 81.915) (width 1.524) (layer F.Cu) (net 14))
 (segment (start 105.055882 80.01) (end 106.960882 81.915) (width 1.524) (layer F.Cu) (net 14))
 (segment (start 96.29 80.01) (end 105.055882 80.01) (width 1.524) (layer F.Cu) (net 14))
 (segment (start 102.125 61.335) (end 99.96 63.5) (width 0.508) (layer F.Cu) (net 13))
 (segment (start 102.625 61.335) (end 102.125 61.335) (width 0.508) (layer F.Cu) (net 13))
 (segment (start 99.96 63.5) (end 92.71 63.5) (width 0.508) (layer F.Cu) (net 13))
 (segment (start 92.71 63.5) (end 90.17 60.96) (width 0.508) (layer F.Cu) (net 13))
 (segment (start 90.245 60.885) (end 90.245 59.055) (width 0.508) (layer F.Cu) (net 13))
 (segment (start 90.17 60.96) (end 90.245 60.885) (width 0.508) (layer F.Cu) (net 13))
 (segment (start 88.9 58.05) (end 87.895 59.055) (width 0.508) (layer F.Cu) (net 13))
 (segment (start 88.9 54.61) (end 88.9 58.05) (width 0.508) (layer F.Cu) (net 13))
 (segment (start 86.055 57.785) (end 86.285 57.555) (width 0.508) (layer F.Cu) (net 12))
 (segment (start 84.527 57.555) (end 86.285 57.555) (width 0.508) (layer F.Cu) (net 12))
 (segment (start 83.076 59.006) (end 84.527 57.555) (width 0.508) (layer F.Cu) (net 12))
 (segment (start 83.076 64.008) (end 83.076 59.006) (width 0.508) (layer F.Cu) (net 12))
 (segment (start 102.125 71.495) (end 99.96 73.66) (width 0.508) (layer F.Cu) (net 17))
 (segment (start 102.625 71.495) (end 102.125 71.495) (width 0.508) (layer F.Cu) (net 17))
 (segment (start 99.96 73.66) (end 92.075 73.66) (width 0.508) (layer F.Cu) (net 17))
 (segment (start 90.17 71.755) (end 90.17 69.215) (width 0.508) (layer F.Cu) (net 17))
 (segment (start 92.075 73.66) (end 90.17 71.755) (width 0.508) (layer F.Cu) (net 17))
 (segment (start 88.9 68.135) (end 87.82 69.215) (width 0.508) (layer F.Cu) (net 17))
 (segment (start 88.9 64.77) (end 88.9 68.135) (width 0.508) (layer F.Cu) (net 17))
 (segment (start 85.98 67.945) (end 86.21 67.715) (width 0.508) (layer F.Cu) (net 19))
 (segment (start 83.185 67.945) (end 85.98 67.945) (width 0.508) (layer F.Cu) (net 19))
 (segment (start 102.09 82.29) (end 100.56 83.82) (width 0.508) (layer F.Cu) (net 15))
 (segment (start 102.59 82.29) (end 102.09 82.29) (width 0.508) (layer F.Cu) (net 15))
 (segment (start 100.56 83.82) (end 92.075 83.82) (width 0.508) (layer F.Cu) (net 15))
 (segment (start 90.245 81.99) (end 90.245 80.01) (width 0.508) (layer F.Cu) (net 15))
 (segment (start 92.075 83.82) (end 90.245 81.99) (width 0.508) (layer F.Cu) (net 15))
 (segment (start 88.755 79.15) (end 87.895 80.01) (width 0.508) (layer F.Cu) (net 15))
 (segment (start 88.755 75.565) (end 88.755 79.15) (width 0.508) (layer F.Cu) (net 15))
 (segment (start 86.13 78.51) (end 83.185 75.565) (width 0.508) (layer F.Cu) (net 18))
 (segment (start 86.285 78.51) (end 86.13 78.51) (width 0.508) (layer F.Cu) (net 18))
 (segment (start 66.04 68.97) (end 66.92 68.97) (width 0.508) (layer F.Cu) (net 5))
 (segment (start 70.7 65.19) (end 70.7 62.23) (width 0.508) (layer F.Cu) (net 5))
 (segment (start 66.92 68.97) (end 70.7 65.19) (width 0.508) (layer F.Cu) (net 5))
 (segment (start 64.135 69.645) (end 64.594 70.104) (width 0.508) (layer F.Cu) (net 2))
 (segment (start 64.135 68.97) (end 64.135 69.645) (width 0.508) (layer F.Cu) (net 2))
 (segment (start 64.594 70.104) (end 64.594 70.182) (width 0.508) (layer F.Cu) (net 2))
 (segment (start 64.594 70.182) (end 64.77 70.358) (width 0.508) (layer F.Cu) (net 2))
 (segment (start 76.2 63.738) (end 76.2 62.23) (width 0.508) (layer F.Cu) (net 2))
 (segment (start 69.58 70.358) (end 76.2 63.738) (width 0.508) (layer F.Cu) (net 2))
 (segment (start 64.77 70.358) (end 69.58 70.358) (width 0.508) (layer F.Cu) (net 2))
 (segment (start 76.874 58.674) (end 78.232 58.674) (width 0.508) (layer F.Cu) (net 2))
 (segment (start 76.2 59.348) (end 76.874 58.674) (width 0.508) (layer F.Cu) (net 2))
 (segment (start 76.2 62.23) (end 76.2 59.348) (width 0.508) (layer F.Cu) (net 2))
 (segment (start 75.1 70.722) (end 80.036 65.786) (width 0.508) (layer F.Cu) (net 10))
 (segment (start 75.1 72.23) (end 75.1 70.722) (width 0.508) (layer F.Cu) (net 10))
 (segment (start 80.036 65.786) (end 80.518 65.786) (width 0.508) (layer F.Cu) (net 10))
 (segment (start 81.026 65.278) (end 81.026 64.008) (width 0.508) (layer F.Cu) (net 10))
 (segment (start 80.518 65.786) (end 81.026 65.278) (width 0.508) (layer F.Cu) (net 10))
 (segment (start 77.3 71.63) (end 80.985 67.945) (width 0.508) (layer F.Cu) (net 9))
 (segment (start 80.985 67.945) (end 81.135 67.945) (width 0.508) (layer F.Cu) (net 9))
 (segment (start 77.3 72.23) (end 77.3 71.63) (width 0.508) (layer F.Cu) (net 9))
 (segment (start 81.135 75.565) (end 80.391 75.565) (width 0.508) (layer F.Cu) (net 11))
 (segment (start 80.391 75.565) (end 78.994 74.168) (width 0.508) (layer F.Cu) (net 11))
 (segment (start 74 73.738) (end 74 72.23) (width 0.508) (layer F.Cu) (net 11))
 (segment (start 74.43 74.168) (end 74 73.738) (width 0.508) (layer F.Cu) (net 11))
 (segment (start 78.994 74.168) (end 74.43 74.168) (width 0.508) (layer F.Cu) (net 11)))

